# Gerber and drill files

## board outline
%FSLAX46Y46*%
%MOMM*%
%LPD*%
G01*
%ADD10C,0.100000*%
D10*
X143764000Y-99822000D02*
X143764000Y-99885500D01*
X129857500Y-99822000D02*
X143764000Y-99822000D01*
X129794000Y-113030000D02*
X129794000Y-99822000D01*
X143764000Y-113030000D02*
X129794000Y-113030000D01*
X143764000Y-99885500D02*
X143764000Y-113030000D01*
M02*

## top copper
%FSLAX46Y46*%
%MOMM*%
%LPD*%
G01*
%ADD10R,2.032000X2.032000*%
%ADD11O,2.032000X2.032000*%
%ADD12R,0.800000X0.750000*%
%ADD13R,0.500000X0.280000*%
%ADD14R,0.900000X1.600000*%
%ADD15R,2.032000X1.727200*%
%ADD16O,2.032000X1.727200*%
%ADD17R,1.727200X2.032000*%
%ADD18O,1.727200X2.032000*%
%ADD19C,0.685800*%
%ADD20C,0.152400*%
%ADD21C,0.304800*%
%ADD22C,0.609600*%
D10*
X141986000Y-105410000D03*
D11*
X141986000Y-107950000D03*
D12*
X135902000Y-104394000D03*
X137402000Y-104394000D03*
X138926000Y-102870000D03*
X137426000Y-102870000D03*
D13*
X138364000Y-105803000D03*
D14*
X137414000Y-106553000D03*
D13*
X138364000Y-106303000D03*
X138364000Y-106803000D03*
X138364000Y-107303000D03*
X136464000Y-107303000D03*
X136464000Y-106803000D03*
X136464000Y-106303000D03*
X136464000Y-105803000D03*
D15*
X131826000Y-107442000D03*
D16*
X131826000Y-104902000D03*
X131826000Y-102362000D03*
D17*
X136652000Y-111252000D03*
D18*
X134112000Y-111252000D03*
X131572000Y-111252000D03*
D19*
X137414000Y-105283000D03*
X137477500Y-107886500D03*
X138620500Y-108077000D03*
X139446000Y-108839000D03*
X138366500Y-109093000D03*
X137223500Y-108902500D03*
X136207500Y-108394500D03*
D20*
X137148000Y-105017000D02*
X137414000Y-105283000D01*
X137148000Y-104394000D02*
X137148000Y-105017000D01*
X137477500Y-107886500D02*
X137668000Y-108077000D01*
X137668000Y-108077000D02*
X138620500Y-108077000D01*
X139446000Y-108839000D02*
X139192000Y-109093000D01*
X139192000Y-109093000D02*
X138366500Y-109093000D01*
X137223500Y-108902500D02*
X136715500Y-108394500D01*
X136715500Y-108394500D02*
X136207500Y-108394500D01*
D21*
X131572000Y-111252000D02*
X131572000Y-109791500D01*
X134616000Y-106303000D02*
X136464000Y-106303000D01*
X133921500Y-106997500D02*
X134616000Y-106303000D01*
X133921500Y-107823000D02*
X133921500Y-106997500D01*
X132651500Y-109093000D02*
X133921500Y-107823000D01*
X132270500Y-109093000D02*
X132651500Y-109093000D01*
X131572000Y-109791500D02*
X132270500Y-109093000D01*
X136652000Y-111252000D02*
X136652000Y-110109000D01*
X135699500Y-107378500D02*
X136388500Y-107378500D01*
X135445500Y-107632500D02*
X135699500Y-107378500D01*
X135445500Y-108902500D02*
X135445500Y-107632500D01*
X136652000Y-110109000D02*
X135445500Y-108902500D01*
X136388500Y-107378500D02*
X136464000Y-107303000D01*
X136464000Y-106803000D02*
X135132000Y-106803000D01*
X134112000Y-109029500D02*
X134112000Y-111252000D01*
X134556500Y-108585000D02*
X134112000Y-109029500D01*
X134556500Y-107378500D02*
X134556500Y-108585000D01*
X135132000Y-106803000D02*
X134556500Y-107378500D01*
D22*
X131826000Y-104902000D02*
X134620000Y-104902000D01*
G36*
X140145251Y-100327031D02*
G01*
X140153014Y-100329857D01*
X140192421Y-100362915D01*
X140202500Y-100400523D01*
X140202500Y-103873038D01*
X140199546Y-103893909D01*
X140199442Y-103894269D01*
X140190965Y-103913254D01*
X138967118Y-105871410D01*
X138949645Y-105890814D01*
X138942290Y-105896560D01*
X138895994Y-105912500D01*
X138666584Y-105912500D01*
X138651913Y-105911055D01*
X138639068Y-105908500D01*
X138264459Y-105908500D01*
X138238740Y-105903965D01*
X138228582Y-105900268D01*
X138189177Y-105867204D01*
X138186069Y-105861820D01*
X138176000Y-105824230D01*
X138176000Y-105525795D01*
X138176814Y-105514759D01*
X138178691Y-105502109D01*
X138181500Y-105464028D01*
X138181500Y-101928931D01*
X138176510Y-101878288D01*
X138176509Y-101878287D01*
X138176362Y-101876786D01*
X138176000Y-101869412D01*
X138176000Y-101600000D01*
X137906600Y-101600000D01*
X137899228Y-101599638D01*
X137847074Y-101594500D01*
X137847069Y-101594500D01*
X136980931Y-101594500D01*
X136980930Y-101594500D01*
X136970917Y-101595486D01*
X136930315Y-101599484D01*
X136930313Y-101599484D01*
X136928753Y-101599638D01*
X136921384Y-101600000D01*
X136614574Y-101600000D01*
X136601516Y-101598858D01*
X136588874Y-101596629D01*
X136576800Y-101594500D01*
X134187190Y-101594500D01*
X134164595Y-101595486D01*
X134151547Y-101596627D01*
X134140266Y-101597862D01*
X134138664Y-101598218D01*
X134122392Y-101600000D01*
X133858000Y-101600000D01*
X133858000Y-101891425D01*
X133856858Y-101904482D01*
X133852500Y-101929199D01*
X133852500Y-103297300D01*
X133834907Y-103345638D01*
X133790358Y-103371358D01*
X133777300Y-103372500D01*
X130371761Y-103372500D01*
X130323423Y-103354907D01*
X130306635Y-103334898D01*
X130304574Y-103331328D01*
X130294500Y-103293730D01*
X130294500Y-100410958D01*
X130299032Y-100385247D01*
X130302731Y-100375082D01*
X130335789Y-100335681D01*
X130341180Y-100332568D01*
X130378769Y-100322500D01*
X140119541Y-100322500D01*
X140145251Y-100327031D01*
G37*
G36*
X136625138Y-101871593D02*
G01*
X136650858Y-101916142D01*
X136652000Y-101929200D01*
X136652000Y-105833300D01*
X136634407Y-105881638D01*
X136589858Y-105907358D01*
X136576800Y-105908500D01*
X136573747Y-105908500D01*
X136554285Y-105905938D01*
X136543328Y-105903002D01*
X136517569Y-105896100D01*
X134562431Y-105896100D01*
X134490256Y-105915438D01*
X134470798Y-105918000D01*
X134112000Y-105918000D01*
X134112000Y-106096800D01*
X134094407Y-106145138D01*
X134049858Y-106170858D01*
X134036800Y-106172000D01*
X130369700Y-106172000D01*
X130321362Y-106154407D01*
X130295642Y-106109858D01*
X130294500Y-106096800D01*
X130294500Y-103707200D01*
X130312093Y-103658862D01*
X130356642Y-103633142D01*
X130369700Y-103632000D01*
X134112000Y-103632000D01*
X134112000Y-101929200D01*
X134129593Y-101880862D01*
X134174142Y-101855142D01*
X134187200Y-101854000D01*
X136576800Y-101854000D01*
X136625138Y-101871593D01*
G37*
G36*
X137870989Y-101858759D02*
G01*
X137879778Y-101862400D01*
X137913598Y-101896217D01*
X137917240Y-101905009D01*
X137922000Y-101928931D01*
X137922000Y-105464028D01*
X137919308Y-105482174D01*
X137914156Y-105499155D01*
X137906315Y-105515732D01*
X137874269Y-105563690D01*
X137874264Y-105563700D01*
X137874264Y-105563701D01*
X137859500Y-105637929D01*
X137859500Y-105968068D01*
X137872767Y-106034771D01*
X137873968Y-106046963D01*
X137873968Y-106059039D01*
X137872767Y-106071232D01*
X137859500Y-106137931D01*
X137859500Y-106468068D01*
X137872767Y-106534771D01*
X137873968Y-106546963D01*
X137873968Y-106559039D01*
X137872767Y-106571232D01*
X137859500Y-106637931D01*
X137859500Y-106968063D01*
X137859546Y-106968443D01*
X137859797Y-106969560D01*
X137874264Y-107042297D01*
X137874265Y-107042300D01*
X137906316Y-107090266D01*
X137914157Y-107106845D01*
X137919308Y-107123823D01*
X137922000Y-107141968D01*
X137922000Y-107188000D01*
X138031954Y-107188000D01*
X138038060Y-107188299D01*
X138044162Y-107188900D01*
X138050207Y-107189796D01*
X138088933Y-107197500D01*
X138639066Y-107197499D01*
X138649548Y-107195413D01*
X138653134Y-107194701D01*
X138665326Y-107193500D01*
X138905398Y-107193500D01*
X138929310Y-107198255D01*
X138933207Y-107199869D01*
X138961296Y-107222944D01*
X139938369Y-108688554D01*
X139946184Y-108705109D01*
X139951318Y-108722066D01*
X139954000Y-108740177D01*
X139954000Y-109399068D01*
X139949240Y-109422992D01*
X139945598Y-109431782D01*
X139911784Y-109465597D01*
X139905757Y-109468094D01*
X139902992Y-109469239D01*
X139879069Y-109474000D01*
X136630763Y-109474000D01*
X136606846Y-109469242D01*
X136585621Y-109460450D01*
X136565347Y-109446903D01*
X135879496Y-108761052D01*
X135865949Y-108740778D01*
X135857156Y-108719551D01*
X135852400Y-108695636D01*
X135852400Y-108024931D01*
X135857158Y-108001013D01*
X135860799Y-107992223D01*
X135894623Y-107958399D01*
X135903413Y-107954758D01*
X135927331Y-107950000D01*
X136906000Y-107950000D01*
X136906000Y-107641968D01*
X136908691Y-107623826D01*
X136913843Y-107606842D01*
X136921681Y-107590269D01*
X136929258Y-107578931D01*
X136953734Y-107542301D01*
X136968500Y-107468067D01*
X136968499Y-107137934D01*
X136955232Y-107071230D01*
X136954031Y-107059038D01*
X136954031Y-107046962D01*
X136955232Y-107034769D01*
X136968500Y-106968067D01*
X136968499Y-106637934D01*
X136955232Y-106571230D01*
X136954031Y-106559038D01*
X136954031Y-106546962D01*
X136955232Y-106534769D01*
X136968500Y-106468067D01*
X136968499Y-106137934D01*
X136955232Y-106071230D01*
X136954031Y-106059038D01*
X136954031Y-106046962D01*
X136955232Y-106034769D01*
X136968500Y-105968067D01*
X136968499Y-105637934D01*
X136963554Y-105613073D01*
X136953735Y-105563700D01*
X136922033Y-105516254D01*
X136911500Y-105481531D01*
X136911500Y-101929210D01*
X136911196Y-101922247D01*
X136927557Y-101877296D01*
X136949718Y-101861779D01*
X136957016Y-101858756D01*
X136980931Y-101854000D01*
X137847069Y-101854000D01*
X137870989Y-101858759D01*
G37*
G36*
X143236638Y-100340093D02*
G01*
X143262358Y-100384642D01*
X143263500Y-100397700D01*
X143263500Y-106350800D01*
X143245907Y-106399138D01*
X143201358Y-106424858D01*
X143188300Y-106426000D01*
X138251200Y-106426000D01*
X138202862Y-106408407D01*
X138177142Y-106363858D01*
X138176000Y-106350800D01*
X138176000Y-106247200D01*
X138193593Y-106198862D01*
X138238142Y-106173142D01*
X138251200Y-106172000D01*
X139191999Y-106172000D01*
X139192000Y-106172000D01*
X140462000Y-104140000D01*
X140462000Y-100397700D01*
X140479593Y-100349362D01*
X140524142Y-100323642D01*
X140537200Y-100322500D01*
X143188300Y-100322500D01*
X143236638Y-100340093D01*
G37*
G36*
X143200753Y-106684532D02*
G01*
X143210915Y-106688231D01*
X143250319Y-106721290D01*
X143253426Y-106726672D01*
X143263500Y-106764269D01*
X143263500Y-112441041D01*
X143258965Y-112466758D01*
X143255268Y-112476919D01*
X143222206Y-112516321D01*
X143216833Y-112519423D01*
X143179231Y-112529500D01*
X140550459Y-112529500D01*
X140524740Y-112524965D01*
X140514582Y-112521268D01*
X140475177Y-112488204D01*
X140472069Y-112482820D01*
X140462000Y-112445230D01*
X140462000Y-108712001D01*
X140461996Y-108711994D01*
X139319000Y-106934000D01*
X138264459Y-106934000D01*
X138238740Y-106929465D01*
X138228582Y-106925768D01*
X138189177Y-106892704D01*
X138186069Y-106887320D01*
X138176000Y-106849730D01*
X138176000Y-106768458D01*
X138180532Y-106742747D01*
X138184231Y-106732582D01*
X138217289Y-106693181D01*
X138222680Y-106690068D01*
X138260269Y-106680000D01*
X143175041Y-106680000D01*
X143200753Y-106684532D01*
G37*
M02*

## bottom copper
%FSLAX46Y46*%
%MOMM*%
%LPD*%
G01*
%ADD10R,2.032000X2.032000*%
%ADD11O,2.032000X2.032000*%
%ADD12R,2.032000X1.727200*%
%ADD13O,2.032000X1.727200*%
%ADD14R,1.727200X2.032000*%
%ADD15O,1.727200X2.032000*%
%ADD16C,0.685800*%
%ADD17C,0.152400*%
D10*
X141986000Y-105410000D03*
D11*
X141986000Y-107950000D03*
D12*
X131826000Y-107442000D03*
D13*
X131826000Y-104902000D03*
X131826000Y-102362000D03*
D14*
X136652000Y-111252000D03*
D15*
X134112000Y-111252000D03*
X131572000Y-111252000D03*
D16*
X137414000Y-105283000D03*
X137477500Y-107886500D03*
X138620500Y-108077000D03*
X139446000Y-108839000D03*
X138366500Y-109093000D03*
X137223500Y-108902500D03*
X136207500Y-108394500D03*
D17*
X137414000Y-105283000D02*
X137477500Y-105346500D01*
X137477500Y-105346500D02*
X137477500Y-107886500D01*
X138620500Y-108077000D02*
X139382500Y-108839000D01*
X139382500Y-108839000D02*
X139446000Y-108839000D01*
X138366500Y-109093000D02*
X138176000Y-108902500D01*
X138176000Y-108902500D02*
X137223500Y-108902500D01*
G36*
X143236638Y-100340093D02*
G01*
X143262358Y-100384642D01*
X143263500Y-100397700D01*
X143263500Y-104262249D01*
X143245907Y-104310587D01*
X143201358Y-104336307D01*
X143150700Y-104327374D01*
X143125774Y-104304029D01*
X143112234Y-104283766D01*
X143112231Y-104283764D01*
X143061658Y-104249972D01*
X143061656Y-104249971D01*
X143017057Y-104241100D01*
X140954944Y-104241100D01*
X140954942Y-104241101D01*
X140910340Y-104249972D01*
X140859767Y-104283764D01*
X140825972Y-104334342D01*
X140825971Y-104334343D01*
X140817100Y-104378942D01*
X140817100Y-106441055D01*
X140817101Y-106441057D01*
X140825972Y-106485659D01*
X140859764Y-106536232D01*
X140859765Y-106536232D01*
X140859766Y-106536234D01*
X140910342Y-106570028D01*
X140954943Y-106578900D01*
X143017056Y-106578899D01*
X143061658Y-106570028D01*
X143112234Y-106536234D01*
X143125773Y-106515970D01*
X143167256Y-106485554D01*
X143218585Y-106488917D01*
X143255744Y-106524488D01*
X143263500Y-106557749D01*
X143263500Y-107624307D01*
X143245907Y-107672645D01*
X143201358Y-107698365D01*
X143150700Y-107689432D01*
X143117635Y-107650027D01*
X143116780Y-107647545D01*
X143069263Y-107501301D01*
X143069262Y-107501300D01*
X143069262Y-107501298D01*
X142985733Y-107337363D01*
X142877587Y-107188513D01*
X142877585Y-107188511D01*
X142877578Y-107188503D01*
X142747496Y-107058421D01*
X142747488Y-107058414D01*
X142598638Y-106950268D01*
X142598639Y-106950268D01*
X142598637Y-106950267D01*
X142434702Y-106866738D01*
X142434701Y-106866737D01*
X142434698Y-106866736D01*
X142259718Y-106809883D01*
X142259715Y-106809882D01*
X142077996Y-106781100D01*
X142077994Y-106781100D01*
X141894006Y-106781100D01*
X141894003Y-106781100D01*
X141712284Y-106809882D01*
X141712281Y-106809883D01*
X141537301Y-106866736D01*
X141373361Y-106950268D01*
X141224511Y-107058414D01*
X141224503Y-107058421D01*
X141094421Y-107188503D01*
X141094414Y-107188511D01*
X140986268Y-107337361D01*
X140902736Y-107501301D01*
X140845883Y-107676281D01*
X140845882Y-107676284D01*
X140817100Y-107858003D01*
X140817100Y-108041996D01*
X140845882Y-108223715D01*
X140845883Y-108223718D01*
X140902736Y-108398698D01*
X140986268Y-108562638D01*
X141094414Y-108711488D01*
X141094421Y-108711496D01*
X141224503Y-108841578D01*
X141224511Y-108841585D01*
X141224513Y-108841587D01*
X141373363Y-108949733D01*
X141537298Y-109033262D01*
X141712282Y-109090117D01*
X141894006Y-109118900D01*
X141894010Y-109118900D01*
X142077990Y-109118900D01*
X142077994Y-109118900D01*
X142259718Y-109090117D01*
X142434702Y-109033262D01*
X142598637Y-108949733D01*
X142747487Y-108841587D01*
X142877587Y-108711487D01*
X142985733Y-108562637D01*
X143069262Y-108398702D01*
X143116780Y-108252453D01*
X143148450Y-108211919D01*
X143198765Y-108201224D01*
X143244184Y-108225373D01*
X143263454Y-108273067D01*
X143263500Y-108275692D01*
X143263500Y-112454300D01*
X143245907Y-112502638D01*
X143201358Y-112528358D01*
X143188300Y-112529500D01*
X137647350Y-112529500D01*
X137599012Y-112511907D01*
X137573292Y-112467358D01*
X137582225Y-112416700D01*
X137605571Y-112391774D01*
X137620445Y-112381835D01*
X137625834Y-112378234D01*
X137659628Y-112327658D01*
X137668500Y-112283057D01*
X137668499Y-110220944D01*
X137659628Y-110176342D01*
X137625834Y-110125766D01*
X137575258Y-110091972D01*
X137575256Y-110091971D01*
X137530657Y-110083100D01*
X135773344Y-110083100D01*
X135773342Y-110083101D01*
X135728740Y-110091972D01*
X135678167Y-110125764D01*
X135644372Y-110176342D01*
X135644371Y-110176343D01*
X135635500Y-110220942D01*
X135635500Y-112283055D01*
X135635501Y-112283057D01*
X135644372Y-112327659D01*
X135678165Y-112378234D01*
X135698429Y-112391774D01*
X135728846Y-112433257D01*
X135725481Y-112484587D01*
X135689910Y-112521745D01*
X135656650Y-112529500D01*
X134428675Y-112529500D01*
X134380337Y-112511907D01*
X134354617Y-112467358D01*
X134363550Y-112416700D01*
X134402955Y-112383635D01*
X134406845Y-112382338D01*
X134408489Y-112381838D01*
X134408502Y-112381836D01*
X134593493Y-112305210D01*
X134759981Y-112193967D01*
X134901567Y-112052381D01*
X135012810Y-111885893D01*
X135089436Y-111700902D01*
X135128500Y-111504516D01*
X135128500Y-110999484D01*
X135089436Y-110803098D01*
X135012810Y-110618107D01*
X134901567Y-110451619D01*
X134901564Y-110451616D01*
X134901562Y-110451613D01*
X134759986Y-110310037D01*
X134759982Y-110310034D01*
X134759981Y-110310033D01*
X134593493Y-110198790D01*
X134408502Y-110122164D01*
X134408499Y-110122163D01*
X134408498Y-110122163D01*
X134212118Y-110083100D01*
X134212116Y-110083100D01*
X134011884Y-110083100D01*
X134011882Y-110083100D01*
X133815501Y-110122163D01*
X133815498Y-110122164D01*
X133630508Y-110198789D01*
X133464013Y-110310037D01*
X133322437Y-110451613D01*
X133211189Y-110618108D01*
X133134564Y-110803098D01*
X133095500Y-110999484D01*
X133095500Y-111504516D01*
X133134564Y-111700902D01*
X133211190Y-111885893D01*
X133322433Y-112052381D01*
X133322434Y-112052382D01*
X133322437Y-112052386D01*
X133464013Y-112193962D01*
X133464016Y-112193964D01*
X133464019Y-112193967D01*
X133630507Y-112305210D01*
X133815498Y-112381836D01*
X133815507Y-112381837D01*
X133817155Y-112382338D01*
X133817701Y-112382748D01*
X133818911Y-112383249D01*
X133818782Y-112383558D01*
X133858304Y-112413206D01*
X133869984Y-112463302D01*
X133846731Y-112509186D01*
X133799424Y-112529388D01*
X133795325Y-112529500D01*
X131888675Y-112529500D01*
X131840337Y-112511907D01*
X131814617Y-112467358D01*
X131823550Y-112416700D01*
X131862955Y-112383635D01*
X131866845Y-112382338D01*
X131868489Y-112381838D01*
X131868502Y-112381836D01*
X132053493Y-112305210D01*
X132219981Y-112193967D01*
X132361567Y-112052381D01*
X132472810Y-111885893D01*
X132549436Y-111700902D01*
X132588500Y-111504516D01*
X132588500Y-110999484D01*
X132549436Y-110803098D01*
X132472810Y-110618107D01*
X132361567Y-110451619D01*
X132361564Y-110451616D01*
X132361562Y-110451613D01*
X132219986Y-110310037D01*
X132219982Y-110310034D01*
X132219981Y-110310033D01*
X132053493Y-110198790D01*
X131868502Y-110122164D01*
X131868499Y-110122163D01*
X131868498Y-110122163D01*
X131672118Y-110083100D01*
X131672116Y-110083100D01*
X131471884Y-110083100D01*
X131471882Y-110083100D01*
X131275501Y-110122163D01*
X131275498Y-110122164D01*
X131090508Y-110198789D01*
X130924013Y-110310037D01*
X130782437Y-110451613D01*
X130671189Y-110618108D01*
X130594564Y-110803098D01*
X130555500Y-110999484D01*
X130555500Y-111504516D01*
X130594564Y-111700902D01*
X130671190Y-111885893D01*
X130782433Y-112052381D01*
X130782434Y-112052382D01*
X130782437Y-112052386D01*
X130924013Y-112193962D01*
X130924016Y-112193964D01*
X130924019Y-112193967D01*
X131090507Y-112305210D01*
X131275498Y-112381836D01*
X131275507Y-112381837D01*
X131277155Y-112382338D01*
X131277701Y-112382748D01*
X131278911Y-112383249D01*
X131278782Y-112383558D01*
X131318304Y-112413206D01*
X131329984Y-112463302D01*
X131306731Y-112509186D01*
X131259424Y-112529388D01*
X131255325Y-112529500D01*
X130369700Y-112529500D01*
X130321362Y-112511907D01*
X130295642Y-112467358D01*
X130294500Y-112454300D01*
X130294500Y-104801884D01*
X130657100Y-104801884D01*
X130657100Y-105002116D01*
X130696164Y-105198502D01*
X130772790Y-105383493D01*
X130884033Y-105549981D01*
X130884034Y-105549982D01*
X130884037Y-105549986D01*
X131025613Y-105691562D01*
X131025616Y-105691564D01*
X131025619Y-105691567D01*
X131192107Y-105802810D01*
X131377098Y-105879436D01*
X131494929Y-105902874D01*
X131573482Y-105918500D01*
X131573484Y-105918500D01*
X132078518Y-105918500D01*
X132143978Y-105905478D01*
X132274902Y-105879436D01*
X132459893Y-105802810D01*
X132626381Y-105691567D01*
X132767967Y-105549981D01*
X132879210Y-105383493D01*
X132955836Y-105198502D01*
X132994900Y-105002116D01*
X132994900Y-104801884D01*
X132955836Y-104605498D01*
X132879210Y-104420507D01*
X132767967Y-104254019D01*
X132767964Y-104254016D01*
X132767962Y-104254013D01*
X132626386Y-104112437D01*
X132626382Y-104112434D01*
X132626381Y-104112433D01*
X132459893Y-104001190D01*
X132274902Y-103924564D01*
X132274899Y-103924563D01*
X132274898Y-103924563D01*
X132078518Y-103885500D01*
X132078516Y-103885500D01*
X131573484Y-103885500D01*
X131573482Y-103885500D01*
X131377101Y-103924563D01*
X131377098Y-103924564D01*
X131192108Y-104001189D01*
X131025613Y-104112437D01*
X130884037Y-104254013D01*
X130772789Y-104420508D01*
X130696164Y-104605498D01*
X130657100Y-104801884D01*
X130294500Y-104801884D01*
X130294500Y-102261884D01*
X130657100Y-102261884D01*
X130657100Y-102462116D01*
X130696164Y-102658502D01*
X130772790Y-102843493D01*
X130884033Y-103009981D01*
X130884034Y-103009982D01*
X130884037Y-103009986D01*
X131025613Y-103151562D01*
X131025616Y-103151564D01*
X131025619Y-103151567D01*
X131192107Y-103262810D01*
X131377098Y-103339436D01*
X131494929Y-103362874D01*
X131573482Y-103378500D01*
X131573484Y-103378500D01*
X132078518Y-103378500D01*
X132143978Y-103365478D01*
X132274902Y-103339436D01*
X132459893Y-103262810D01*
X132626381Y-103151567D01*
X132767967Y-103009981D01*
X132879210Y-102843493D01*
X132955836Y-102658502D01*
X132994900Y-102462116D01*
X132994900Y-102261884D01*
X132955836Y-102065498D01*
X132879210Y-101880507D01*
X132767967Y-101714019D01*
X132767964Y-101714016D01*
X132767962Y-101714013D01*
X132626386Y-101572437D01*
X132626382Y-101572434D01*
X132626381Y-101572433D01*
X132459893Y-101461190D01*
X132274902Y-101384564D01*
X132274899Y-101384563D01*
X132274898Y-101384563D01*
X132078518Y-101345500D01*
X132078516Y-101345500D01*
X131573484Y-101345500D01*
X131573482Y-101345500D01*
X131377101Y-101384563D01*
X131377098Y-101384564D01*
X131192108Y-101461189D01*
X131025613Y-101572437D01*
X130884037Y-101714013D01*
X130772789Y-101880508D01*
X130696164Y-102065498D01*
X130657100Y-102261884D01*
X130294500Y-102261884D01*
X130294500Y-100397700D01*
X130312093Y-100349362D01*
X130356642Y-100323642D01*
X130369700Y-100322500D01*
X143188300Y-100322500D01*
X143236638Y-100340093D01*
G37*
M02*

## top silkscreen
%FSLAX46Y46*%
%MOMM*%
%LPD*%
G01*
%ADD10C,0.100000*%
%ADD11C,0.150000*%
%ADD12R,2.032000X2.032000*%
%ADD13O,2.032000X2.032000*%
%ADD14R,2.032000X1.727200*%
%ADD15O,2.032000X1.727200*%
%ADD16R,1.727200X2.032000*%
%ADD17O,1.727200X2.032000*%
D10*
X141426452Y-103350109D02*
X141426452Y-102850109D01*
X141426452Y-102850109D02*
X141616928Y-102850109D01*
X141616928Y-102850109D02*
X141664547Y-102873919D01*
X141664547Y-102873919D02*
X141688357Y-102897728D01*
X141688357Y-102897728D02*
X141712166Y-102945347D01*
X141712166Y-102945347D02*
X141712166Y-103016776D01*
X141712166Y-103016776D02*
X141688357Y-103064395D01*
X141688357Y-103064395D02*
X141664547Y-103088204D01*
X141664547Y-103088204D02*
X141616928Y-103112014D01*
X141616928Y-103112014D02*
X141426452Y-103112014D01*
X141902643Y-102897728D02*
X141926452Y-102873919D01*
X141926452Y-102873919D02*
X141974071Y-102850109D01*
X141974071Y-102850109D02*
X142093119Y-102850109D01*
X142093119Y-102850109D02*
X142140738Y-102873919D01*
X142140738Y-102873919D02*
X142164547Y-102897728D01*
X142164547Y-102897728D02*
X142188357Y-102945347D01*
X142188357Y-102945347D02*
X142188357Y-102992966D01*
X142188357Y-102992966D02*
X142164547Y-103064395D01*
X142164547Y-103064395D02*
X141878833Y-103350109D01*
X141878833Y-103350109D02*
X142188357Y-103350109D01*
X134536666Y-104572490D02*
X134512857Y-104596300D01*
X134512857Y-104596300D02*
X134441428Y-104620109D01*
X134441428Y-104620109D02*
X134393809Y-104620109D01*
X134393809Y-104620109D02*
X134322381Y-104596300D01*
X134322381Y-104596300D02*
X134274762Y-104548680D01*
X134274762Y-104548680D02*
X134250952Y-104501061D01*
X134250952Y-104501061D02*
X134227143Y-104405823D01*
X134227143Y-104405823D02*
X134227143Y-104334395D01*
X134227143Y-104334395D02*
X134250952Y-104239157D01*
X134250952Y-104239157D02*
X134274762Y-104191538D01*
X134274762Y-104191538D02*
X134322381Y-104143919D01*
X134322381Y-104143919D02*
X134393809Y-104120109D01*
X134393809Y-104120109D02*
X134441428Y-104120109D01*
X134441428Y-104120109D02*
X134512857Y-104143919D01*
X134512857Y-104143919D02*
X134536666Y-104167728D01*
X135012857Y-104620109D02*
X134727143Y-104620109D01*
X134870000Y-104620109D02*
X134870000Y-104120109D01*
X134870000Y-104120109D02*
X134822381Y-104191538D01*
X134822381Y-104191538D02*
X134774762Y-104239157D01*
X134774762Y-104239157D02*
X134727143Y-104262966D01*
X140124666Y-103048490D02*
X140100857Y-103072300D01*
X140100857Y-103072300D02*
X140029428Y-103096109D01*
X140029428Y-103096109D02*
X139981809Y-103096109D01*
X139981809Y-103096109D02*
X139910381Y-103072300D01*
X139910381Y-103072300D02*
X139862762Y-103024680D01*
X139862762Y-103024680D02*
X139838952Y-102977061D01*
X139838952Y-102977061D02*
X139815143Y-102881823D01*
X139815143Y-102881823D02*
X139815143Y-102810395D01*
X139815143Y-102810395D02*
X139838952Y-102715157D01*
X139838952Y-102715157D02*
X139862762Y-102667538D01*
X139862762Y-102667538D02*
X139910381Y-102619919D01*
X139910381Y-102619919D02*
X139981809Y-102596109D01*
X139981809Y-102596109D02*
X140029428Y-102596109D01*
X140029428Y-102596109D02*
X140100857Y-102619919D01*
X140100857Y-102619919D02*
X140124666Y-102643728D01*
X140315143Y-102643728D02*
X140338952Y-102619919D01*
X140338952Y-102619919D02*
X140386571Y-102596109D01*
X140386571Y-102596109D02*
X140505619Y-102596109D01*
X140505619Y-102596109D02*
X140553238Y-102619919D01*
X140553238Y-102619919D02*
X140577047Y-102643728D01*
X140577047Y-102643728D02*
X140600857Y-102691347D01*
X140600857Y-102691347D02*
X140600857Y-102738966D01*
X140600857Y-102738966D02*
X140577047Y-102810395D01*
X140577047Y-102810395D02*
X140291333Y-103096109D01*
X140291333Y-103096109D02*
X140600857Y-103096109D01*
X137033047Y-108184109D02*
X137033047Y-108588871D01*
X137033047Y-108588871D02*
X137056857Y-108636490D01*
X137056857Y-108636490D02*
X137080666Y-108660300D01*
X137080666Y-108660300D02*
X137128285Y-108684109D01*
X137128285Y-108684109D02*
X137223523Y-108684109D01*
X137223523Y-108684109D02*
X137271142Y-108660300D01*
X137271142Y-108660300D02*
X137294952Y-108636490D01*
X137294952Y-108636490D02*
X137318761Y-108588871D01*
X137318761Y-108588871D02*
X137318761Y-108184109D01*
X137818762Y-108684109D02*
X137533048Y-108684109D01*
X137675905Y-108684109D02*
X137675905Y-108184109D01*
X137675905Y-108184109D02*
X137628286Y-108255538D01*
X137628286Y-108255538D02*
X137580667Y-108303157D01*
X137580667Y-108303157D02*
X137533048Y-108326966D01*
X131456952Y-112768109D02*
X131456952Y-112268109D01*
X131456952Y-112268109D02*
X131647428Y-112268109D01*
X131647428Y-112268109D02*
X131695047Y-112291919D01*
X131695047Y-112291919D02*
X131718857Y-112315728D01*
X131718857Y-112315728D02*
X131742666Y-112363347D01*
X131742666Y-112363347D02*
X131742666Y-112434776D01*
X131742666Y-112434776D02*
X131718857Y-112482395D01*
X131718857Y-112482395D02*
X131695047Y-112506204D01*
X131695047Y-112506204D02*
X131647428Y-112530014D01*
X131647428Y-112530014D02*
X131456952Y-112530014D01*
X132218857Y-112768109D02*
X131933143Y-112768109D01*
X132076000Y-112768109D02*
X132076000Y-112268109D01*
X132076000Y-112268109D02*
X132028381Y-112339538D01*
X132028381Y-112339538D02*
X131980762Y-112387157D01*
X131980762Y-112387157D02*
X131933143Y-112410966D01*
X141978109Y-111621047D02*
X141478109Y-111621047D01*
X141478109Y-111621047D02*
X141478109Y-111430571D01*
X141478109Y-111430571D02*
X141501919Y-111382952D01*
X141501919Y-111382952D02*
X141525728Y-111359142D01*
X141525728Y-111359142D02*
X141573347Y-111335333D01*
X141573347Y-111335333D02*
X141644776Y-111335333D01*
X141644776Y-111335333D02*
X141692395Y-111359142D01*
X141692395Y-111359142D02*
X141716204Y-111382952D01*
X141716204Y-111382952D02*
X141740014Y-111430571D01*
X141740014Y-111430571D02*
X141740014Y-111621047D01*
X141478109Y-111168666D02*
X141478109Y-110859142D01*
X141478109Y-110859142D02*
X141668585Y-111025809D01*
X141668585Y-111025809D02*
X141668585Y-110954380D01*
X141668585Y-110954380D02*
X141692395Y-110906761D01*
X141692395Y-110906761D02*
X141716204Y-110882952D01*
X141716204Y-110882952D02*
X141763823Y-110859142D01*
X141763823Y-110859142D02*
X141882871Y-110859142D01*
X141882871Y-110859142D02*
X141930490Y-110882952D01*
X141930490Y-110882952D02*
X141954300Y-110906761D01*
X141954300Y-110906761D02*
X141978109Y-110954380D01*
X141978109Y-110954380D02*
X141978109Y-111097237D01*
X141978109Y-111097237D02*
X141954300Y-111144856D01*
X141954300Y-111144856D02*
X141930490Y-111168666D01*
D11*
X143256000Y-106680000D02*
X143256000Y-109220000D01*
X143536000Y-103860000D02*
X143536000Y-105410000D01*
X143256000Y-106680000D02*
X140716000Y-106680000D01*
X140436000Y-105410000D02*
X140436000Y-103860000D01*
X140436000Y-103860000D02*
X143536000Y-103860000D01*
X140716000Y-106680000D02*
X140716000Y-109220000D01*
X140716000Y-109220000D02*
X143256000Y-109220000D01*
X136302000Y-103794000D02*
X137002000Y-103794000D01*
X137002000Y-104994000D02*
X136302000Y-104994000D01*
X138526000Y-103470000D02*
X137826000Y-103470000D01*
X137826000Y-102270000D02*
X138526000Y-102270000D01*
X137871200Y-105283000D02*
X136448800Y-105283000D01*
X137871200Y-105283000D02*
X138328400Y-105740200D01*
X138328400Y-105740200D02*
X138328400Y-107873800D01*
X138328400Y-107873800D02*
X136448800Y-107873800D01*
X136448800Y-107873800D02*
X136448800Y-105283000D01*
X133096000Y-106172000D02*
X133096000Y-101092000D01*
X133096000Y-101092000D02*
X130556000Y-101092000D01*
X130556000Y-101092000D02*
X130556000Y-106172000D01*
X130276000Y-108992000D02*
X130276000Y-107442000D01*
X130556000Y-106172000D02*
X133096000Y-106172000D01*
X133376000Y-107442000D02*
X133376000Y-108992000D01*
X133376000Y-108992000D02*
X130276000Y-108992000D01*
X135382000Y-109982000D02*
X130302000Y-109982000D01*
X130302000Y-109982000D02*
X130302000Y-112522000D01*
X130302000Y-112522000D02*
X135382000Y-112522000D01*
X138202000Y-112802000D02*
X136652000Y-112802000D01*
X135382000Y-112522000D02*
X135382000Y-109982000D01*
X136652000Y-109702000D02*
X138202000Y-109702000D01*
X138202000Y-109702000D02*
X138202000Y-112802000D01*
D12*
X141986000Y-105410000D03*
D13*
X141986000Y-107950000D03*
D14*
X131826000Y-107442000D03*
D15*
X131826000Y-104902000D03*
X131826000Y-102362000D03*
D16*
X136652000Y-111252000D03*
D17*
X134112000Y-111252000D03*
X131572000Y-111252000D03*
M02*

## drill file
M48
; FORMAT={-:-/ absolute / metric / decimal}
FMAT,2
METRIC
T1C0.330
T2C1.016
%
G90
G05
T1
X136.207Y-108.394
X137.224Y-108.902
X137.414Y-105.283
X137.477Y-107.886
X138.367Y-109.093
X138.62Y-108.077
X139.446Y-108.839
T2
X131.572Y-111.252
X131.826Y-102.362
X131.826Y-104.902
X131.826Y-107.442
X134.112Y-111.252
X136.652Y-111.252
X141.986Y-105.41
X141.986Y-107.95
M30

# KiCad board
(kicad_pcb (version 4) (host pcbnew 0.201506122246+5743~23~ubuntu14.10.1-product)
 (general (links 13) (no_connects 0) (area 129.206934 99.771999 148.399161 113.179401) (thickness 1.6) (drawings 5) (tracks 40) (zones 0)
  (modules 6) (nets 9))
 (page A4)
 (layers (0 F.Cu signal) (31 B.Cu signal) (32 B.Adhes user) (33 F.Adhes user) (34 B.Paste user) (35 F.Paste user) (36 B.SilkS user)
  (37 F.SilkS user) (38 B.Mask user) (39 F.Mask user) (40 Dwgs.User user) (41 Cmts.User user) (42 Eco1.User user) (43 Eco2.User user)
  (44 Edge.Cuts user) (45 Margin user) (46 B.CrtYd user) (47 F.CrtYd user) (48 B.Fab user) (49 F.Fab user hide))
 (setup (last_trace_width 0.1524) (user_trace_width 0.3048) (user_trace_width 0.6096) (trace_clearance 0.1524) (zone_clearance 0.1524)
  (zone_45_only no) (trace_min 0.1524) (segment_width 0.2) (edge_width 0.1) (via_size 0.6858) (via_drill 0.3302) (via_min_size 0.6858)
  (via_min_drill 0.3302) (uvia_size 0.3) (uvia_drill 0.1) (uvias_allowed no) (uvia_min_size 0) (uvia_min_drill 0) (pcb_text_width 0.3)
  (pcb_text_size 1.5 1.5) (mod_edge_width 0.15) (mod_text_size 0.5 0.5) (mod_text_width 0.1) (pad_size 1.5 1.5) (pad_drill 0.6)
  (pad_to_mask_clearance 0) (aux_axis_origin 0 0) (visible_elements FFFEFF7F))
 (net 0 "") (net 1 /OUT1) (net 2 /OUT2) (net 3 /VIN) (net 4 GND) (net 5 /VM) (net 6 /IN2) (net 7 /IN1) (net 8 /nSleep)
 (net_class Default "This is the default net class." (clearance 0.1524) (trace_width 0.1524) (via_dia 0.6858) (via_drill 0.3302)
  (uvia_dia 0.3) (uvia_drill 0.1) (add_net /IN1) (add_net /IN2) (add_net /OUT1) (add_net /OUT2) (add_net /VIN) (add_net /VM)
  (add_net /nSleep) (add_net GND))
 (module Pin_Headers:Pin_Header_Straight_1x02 (layer F.Cu) (at 141.986 105.41)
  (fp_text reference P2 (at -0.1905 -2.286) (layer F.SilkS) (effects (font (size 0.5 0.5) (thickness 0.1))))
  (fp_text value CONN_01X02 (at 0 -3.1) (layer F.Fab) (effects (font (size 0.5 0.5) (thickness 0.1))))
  (fp_line (start 1.27 1.27) (end 1.27 3.81) (layer F.SilkS) (width 0.15))
  (fp_line (start 1.55 -1.55) (end 1.55 0) (layer F.SilkS) (width 0.15))
  (fp_line (start 1.27 1.27) (end -1.27 1.27) (layer F.SilkS) (width 0.15))
  (fp_line (start -1.55 0) (end -1.55 -1.55) (layer F.SilkS) (width 0.15))
  (fp_line (start -1.55 -1.55) (end 1.55 -1.55) (layer F.SilkS) (width 0.15))
  (fp_line (start -1.27 1.27) (end -1.27 3.81) (layer F.SilkS) (width 0.15))
  (fp_line (start -1.27 3.81) (end 1.27 3.81) (layer F.SilkS) (width 0.15))
  (pad 1 thru_hole rect (at 0 0) (size 2.032 2.032) (drill 1.016) (layers *.Cu *.Mask F.SilkS) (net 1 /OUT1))
  (pad 2 thru_hole oval (at 0 2.54) (size 2.032 2.032) (drill 1.016) (layers *.Cu *.Mask F.SilkS) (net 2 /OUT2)))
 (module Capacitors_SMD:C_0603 (layer F.Cu) (at 136.652 104.394)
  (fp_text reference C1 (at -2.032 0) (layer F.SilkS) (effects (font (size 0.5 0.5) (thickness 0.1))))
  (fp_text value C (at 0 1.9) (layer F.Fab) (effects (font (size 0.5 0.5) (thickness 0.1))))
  (fp_line (start -0.35 -0.6) (end 0.35 -0.6) (layer F.SilkS) (width 0.15))
  (fp_line (start 0.35 0.6) (end -0.35 0.6) (layer F.SilkS) (width 0.15))
  (pad 1 smd rect (at -0.75 0) (size 0.8 0.75) (layers F.Cu F.Paste F.Mask) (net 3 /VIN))
  (pad 2 smd rect (at 0.75 0) (size 0.8 0.75) (layers F.Cu F.Paste F.Mask) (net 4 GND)))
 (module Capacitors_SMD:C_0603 (layer F.Cu) (at 138.176 102.87 180)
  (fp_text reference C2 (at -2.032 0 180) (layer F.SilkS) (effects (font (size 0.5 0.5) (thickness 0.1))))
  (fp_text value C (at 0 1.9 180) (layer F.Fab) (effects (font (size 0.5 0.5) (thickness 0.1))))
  (fp_line (start -0.35 -0.6) (end 0.35 -0.6) (layer F.SilkS) (width 0.15))
  (fp_line (start 0.35 0.6) (end -0.35 0.6) (layer F.SilkS) (width 0.15))
  (pad 1 smd rect (at -0.75 0 180) (size 0.8 0.75) (layers F.Cu F.Paste F.Mask) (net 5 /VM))
  (pad 2 smd rect (at 0.75 0 180) (size 0.8 0.75) (layers F.Cu F.Paste F.Mask) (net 4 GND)))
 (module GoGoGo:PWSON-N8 (layer F.Cu) (at 137.414 106.553 270)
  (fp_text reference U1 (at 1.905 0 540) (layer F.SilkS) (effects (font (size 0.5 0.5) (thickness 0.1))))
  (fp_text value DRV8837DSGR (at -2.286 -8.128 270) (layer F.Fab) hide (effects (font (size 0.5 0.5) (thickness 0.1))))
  (fp_line (start -1.27 -0.4572) (end -1.27 0.9652) (layer F.SilkS) (width 0.15))
  (fp_line (start -1.27 -0.4572) (end -0.8128 -0.9144) (layer F.SilkS) (width 0.15))
  (fp_line (start -0.8128 -0.9144) (end 1.3208 -0.9144) (layer F.SilkS) (width 0.15))
  (fp_line (start 1.3208 -0.9144) (end 1.3208 0.9652) (layer F.SilkS) (width 0.15))
  (fp_line (start 1.3208 0.9652) (end -1.27 0.9652) (layer F.SilkS) (width 0.15))
  (pad 1 smd rect (at -0.75 -0.95 270) (size 0.28 0.5) (layers F.Cu F.Paste F.Mask) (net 5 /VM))
  (pad 4 smd rect (at 0 0 270) (size 1.6 0.9) (layers F.Cu F.Paste F.Mask) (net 4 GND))
  (pad 2 smd rect (at -0.25 -0.95 270) (size 0.28 0.5) (layers F.Cu F.Paste F.Mask) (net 1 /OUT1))
  (pad 3 smd rect (at 0.25 -0.95 270) (size 0.28 0.5) (layers F.Cu F.Paste F.Mask) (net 2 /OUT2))
  (pad 4 smd rect (at 0.75 -0.95 270) (size 0.28 0.5) (layers F.Cu F.Paste F.Mask) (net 4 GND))
  (pad 5 smd rect (at 0.75 0.95 270) (size 0.28 0.5) (layers F.Cu F.Paste F.Mask) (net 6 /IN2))
  (pad 6 smd rect (at 0.25 0.95 270) (size 0.28 0.5) (layers F.Cu F.Paste F.Mask) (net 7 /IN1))
  (pad 7 smd rect (at -0.25 0.95 270) (size 0.28 0.5) (layers F.Cu F.Paste F.Mask) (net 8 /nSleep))
  (pad 8 smd rect (at -0.75 0.95 270) (size 0.28 0.5) (layers F.Cu F.Paste F.Mask) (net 3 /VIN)))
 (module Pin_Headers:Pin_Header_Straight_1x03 (layer F.Cu) (at 131.826 107.442 180)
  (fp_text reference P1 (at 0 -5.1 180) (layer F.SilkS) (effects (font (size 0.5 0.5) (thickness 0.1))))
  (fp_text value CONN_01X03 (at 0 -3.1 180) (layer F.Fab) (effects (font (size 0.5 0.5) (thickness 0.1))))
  (fp_line (start -1.27 1.27) (end -1.27 6.35) (layer F.SilkS) (width 0.15))
  (fp_line (start -1.27 6.35) (end 1.27 6.35) (layer F.SilkS) (width 0.15))
  (fp_line (start 1.27 6.35) (end 1.27 1.27) (layer F.SilkS) (width 0.15))
  (fp_line (start 1.55 -1.55) (end 1.55 0) (layer F.SilkS) (width 0.15))
  (fp_line (start 1.27 1.27) (end -1.27 1.27) (layer F.SilkS) (width 0.15))
  (fp_line (start -1.55 0) (end -1.55 -1.55) (layer F.SilkS) (width 0.15))
  (fp_line (start -1.55 -1.55) (end 1.55 -1.55) (layer F.SilkS) (width 0.15))
  (pad 1 thru_hole rect (at 0 0 180) (size 2.032 1.7272) (drill 1.016) (layers *.Cu *.Mask F.SilkS) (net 4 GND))
  (pad 2 thru_hole oval (at 0 2.54 180) (size 2.032 1.7272) (drill 1.016) (layers *.Cu *.Mask F.SilkS) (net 3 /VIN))
  (pad 3 thru_hole oval (at 0 5.08 180) (size 2.032 1.7272) (drill 1.016) (layers *.Cu *.Mask F.SilkS) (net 5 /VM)))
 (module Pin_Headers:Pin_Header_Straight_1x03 (layer F.Cu) (at 136.652 111.252 270)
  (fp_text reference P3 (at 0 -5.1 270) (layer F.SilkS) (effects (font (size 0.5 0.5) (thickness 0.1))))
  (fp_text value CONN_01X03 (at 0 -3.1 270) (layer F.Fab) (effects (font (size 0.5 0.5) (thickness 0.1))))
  (fp_line (start -1.27 1.27) (end -1.27 6.35) (layer F.SilkS) (width 0.15))
  (fp_line (start -1.27 6.35) (end 1.27 6.35) (layer F.SilkS) (width 0.15))
  (fp_line (start 1.27 6.35) (end 1.27 1.27) (layer F.SilkS) (width 0.15))
  (fp_line (start 1.55 -1.55) (end 1.55 0) (layer F.SilkS) (width 0.15))
  (fp_line (start 1.27 1.27) (end -1.27 1.27) (layer F.SilkS) (width 0.15))
  (fp_line (start -1.55 0) (end -1.55 -1.55) (layer F.SilkS) (width 0.15))
  (fp_line (start -1.55 -1.55) (end 1.55 -1.55) (layer F.SilkS) (width 0.15))
  (pad 1 thru_hole rect (at 0 0 270) (size 2.032 1.7272) (drill 1.016) (layers *.Cu *.Mask F.SilkS) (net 6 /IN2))
  (pad 2 thru_hole oval (at 0 2.54 270) (size 2.032 1.7272) (drill 1.016) (layers *.Cu *.Mask F.SilkS) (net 7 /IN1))
  (pad 3 thru_hole oval (at 0 5.08 270) (size 2.032 1.7272) (drill 1.016) (layers *.Cu *.Mask F.SilkS) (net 8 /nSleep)))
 (gr_line (start 143.764 99.822) (end 143.764 99.8855) (angle 90) (layer Edge.Cuts) (width 0.1))
 (gr_line (start 129.8575 99.822) (end 143.764 99.822) (angle 90) (layer Edge.Cuts) (width 0.1))
 (gr_line (start 129.794 113.03) (end 129.794 99.822) (angle 90) (layer Edge.Cuts) (width 0.1))
 (gr_line (start 143.764 113.03) (end 129.794 113.03) (angle 90) (layer Edge.Cuts) (width 0.1))
 (gr_line (start 143.764 99.8855) (end 143.764 113.03) (angle 90) (layer Edge.Cuts) (width 0.1))
 (segment (start 137.414 105.283) (end 137.4775 105.3465) (width 0.1524) (layer B.Cu) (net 4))
 (via (at 137.414 105.283) (size 0.6858) (layers F.Cu B.Cu) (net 4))
 (segment (start 137.148 105.017) (end 137.414 105.283) (width 0.1524) (layer F.Cu) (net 4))
 (segment (start 137.148 104.394) (end 137.148 105.017) (width 0.1524) (layer F.Cu) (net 4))
 (segment (start 137.4775 105.3465) (end 137.4775 107.8865) (width 0.1524) (layer B.Cu) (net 4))
 (via (at 137.4775 107.8865) (size 0.6858) (layers F.Cu B.Cu) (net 4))
 (segment (start 137.4775 107.8865) (end 137.668 108.077) (width 0.1524) (layer F.Cu) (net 4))
 (segment (start 137.668 108.077) (end 138.6205 108.077) (width 0.1524) (layer F.Cu) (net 4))
 (via (at 138.6205 108.077) (size 0.6858) (layers F.Cu B.Cu) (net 4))
 (segment (start 138.6205 108.077) (end 139.3825 108.839) (width 0.1524) (layer B.Cu) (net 4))
 (segment (start 139.3825 108.839) (end 139.446 108.839) (width 0.1524) (layer B.Cu) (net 4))
 (via (at 139.446 108.839) (size 0.6858) (layers F.Cu B.Cu) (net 4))
 (segment (start 139.446 108.839) (end 139.192 109.093) (width 0.1524) (layer F.Cu) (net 4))
 (segment (start 139.192 109.093) (end 138.3665 109.093) (width 0.1524) (layer F.Cu) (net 4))
 (via (at 138.3665 109.093) (size 0.6858) (layers F.Cu B.Cu) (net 4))
 (segment (start 138.3665 109.093) (end 138.176 108.9025) (width 0.1524) (layer B.Cu) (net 4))
 (segment (start 138.176 108.9025) (end 137.2235 108.9025) (width 0.1524) (layer B.Cu) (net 4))
 (via (at 137.2235 108.9025) (size 0.6858) (layers F.Cu B.Cu) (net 4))
 (segment (start 137.2235 108.9025) (end 136.7155 108.3945) (width 0.1524) (layer F.Cu) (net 4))
 (segment (start 136.7155 108.3945) (end 136.2075 108.3945) (width 0.1524) (layer F.Cu) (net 4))
 (via (at 136.2075 108.3945) (size 0.6858) (layers F.Cu B.Cu) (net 4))
 (segment (start 131.572 111.252) (end 131.572 109.7915) (width 0.3048) (layer F.Cu) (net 8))
 (segment (start 134.616 106.303) (end 136.464 106.303) (width 0.3048) (layer F.Cu) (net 8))
 (segment (start 133.9215 106.9975) (end 134.616 106.303) (width 0.3048) (layer F.Cu) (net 8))
 (segment (start 133.9215 107.823) (end 133.9215 106.9975) (width 0.3048) (layer F.Cu) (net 8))
 (segment (start 132.6515 109.093) (end 133.9215 107.823) (width 0.3048) (layer F.Cu) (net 8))
 (segment (start 132.2705 109.093) (end 132.6515 109.093) (width 0.3048) (layer F.Cu) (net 8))
 (segment (start 131.572 109.7915) (end 132.2705 109.093) (width 0.3048) (layer F.Cu) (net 8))
 (segment (start 136.652 111.252) (end 136.652 110.109) (width 0.3048) (layer F.Cu) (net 6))
 (segment (start 135.6995 107.3785) (end 136.3885 107.3785) (width 0.3048) (layer F.Cu) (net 6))
 (segment (start 135.4455 107.6325) (end 135.6995 107.3785) (width 0.3048) (layer F.Cu) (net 6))
 (segment (start 135.4455 108.9025) (end 135.4455 107.6325) (width 0.3048) (layer F.Cu) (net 6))
 (segment (start 136.652 110.109) (end 135.4455 108.9025) (width 0.3048) (layer F.Cu) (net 6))
 (segment (start 136.3885 107.3785) (end 136.464 107.303) (width 0.3048) (layer F.Cu) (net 6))
 (segment (start 136.464 106.803) (end 135.132 106.803) (width 0.3048) (layer F.Cu) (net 7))
 (segment (start 134.112 109.0295) (end 134.112 111.252) (width 0.3048) (layer F.Cu) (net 7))
 (segment (start 134.5565 108.585) (end 134.112 109.0295) (width 0.3048) (layer F.Cu) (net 7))
 (segment (start 134.5565 107.3785) (end 134.5565 108.585) (width 0.3048) (layer F.Cu) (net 7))
 (segment (start 135.132 106.803) (end 134.5565 107.3785) (width 0.3048) (layer F.Cu) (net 7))
 (segment (start 131.826 104.902) (end 134.62 104.902) (width 0.6096) (layer F.Cu) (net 3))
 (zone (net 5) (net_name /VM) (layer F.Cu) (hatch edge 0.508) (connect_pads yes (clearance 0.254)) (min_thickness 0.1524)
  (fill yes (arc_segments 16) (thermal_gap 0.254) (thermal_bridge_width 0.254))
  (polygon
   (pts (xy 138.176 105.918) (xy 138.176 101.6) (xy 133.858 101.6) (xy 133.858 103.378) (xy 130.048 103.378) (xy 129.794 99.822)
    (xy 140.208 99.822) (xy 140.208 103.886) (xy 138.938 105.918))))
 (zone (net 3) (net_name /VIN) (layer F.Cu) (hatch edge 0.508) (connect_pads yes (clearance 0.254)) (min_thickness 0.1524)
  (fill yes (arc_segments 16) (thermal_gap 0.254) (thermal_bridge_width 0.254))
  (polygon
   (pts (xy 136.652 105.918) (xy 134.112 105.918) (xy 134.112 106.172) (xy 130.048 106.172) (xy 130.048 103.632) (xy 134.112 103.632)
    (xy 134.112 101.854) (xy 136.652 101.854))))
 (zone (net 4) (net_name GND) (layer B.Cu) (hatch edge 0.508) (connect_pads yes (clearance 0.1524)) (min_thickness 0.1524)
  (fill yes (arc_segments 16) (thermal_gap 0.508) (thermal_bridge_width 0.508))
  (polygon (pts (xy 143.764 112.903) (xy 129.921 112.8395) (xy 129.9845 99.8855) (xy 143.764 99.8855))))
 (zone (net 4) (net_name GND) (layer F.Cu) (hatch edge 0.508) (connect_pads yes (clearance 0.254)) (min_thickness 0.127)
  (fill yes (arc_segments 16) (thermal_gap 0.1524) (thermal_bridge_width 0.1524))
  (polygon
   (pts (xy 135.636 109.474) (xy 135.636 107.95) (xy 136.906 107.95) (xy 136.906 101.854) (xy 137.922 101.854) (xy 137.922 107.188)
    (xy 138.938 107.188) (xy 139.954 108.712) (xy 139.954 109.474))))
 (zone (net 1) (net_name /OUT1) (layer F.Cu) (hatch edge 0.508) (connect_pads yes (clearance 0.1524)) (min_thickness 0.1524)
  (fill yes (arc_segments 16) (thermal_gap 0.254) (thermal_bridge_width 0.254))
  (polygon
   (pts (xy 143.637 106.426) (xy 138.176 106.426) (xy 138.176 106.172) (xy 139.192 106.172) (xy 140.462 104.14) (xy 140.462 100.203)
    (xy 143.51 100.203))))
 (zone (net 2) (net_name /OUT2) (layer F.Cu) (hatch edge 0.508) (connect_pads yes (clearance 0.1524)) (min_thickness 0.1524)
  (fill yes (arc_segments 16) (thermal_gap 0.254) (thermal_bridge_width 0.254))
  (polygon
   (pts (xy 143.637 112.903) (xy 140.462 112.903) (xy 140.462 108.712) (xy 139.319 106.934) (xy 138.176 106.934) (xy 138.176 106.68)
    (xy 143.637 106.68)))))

